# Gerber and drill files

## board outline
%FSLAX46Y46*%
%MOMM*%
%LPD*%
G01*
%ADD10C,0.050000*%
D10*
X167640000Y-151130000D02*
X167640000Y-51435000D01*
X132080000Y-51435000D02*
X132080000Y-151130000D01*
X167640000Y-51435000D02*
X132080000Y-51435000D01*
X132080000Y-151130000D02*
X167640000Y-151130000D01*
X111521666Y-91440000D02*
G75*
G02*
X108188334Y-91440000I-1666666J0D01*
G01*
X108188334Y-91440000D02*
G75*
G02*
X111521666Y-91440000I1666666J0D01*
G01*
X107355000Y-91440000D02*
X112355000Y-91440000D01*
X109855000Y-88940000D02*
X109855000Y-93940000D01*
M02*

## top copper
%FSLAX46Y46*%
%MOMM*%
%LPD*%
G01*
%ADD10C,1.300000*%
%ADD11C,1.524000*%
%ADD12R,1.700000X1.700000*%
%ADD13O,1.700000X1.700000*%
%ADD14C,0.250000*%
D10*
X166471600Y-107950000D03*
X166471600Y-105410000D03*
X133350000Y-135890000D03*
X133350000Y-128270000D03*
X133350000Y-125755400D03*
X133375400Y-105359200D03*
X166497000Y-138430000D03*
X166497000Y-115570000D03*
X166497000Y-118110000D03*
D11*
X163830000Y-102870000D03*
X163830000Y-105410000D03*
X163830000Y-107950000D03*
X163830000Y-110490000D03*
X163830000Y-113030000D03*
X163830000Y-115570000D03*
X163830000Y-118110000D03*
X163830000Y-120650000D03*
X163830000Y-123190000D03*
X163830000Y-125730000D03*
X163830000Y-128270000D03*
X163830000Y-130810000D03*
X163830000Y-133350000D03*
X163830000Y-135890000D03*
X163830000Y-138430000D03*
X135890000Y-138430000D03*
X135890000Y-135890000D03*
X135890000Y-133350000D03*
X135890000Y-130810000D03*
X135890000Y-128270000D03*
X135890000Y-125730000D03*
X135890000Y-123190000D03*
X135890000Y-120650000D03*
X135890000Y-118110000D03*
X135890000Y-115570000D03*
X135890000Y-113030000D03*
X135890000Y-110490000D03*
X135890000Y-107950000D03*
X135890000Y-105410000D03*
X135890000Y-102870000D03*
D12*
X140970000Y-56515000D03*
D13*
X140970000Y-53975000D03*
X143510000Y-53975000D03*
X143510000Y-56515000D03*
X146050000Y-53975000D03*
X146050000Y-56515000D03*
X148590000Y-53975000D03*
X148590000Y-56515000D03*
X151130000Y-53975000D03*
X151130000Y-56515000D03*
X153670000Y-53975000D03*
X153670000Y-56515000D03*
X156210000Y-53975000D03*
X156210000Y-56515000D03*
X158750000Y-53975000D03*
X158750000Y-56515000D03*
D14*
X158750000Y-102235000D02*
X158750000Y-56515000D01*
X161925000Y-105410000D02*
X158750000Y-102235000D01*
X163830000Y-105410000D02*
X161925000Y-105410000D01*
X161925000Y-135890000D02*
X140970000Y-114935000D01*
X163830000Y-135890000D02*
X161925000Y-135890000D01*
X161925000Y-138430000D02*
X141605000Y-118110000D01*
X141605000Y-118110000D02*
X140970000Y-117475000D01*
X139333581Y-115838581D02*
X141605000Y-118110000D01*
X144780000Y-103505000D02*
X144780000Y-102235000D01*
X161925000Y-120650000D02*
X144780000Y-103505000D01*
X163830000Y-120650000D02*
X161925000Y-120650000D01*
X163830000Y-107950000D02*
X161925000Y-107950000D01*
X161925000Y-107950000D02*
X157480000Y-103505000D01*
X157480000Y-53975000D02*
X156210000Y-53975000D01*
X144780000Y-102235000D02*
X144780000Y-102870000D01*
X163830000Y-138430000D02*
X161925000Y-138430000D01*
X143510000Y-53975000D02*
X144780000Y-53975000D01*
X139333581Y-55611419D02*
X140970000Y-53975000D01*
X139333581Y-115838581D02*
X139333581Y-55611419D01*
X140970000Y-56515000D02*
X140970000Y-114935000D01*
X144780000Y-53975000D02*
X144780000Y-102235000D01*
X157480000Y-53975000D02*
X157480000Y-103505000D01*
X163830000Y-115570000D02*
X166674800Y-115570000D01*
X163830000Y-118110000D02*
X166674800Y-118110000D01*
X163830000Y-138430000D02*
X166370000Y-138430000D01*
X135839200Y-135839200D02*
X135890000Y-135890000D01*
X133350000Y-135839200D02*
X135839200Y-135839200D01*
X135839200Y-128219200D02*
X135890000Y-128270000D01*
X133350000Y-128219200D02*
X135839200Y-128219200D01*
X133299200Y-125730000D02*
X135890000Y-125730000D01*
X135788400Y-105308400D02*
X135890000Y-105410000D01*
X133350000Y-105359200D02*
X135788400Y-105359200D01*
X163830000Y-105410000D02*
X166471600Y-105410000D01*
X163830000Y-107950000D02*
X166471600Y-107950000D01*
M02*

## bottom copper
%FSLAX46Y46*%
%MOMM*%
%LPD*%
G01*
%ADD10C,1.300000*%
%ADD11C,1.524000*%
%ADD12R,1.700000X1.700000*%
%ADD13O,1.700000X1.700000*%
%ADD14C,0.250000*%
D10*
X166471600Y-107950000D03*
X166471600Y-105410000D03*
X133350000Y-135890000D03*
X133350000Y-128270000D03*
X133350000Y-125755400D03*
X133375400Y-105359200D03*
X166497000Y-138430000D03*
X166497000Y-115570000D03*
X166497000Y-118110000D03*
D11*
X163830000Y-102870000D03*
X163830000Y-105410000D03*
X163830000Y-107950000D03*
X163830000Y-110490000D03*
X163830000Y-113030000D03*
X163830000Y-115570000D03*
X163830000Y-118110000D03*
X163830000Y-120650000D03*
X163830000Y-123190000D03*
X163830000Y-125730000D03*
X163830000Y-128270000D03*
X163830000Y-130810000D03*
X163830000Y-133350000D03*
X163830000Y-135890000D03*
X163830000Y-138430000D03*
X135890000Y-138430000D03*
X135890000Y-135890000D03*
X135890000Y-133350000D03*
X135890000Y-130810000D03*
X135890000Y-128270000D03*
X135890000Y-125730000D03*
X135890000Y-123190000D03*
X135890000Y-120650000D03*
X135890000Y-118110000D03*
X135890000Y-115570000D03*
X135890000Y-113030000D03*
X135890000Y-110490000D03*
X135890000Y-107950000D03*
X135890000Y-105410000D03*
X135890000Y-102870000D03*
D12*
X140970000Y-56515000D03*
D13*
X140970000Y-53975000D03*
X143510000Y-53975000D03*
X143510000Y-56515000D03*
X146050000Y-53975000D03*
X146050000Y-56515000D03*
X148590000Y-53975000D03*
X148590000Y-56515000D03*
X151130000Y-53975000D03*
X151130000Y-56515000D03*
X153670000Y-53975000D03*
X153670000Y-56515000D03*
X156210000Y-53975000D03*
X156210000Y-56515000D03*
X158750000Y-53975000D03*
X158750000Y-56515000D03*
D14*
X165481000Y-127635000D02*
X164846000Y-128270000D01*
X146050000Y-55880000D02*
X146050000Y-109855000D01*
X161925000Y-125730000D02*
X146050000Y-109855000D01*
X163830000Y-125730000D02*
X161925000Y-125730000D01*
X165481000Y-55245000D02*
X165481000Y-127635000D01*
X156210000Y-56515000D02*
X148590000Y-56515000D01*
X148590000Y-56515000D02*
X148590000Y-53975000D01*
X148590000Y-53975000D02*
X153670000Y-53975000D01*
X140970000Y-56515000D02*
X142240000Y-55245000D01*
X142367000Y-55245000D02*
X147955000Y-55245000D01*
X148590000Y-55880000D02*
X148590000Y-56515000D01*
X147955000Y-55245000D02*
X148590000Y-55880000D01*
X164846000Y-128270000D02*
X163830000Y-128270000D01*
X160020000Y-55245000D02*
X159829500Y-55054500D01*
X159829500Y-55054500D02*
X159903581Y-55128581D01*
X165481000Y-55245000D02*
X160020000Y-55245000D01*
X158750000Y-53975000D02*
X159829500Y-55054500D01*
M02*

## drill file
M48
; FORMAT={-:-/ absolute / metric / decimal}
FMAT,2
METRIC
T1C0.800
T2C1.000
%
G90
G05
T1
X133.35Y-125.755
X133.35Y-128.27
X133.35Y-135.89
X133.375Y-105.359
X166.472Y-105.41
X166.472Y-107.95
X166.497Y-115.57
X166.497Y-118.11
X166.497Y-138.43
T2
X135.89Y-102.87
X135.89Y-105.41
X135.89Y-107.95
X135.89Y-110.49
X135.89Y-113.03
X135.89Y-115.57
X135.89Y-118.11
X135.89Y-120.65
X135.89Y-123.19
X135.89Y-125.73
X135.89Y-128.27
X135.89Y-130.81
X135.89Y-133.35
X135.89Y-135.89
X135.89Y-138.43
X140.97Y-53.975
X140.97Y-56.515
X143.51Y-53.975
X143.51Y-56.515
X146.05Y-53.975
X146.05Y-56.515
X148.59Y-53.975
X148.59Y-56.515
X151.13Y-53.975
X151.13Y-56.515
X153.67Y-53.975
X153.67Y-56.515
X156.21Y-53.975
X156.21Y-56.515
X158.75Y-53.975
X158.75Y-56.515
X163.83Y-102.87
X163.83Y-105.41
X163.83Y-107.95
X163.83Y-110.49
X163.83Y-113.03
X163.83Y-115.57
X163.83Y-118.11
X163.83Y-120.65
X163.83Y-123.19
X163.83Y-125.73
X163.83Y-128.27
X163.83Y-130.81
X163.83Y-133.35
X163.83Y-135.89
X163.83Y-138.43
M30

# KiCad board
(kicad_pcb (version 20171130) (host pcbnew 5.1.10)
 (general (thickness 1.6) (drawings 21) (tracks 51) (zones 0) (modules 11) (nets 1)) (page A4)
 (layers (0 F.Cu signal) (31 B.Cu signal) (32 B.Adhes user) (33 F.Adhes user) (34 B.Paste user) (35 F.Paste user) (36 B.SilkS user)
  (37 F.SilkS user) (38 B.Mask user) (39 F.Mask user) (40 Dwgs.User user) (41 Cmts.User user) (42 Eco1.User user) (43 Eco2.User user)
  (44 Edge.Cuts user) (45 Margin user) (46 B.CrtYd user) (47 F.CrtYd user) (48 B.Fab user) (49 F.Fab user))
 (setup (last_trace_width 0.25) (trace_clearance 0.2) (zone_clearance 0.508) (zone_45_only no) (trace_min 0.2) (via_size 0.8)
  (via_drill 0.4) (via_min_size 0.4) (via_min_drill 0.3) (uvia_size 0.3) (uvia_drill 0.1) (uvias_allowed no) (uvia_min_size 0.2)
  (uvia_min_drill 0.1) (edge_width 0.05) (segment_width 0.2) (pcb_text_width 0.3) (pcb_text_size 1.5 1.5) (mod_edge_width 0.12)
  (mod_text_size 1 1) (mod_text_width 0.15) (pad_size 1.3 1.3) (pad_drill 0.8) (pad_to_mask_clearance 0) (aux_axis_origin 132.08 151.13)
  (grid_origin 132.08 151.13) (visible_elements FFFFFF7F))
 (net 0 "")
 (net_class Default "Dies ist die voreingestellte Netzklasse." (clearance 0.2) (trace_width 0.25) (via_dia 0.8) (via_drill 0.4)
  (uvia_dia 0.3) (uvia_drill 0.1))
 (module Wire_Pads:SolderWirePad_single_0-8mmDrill (layer F.Cu) (at 166.4716 107.95)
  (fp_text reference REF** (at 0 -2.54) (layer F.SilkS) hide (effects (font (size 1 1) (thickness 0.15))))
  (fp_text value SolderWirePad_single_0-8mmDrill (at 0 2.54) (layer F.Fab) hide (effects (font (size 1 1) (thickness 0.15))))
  (pad 1 thru_hole circle (at 0 0) (size 1.3 1.3) (drill 0.8) (layers *.Cu *.Mask)))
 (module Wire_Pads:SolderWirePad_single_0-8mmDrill (layer F.Cu) (at 166.4716 105.41)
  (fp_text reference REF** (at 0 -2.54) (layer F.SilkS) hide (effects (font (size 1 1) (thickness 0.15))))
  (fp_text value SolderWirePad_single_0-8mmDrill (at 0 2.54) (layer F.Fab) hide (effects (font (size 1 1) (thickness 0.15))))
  (pad 1 thru_hole circle (at 0 0) (size 1.3 1.3) (drill 0.8) (layers *.Cu *.Mask)))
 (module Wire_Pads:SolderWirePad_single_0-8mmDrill (layer F.Cu) (at 133.35 135.89)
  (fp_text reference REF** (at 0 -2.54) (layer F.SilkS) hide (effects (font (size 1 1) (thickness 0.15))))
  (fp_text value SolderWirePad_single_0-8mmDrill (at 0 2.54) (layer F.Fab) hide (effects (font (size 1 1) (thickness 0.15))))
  (pad 1 thru_hole circle (at 0 0) (size 1.3 1.3) (drill 0.8) (layers *.Cu *.Mask)))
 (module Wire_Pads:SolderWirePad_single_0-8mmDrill (layer F.Cu) (at 133.35 128.27)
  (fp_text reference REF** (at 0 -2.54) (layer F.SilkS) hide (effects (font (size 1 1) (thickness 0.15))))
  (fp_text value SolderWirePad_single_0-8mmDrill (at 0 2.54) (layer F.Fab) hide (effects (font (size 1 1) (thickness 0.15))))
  (pad 1 thru_hole circle (at 0 0) (size 1.3 1.3) (drill 0.8) (layers *.Cu *.Mask)))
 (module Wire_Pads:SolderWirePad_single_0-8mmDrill (layer F.Cu) (at 133.35 125.7554)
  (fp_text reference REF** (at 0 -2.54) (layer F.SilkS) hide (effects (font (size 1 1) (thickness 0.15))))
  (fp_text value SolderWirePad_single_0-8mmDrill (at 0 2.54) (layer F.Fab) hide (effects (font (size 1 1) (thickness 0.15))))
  (pad 1 thru_hole circle (at 0 0) (size 1.3 1.3) (drill 0.8) (layers *.Cu *.Mask)))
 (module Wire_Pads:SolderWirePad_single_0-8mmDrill (layer F.Cu) (at 133.3754 105.3592)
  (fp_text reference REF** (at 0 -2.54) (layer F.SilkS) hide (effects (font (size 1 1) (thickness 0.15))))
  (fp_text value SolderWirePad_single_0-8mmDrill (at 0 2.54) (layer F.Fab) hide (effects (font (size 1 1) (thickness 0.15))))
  (pad 1 thru_hole circle (at 0 0) (size 1.3 1.3) (drill 0.8) (layers *.Cu *.Mask)))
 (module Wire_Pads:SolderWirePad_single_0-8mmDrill (layer F.Cu) (at 166.497 138.43)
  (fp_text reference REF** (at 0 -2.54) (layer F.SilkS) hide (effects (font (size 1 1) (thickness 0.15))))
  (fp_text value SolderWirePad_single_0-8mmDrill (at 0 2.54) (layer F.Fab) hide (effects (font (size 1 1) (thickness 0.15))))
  (pad 1 thru_hole circle (at 0 0) (size 1.3 1.3) (drill 0.8) (layers *.Cu *.Mask)))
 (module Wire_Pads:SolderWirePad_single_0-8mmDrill (layer F.Cu) (at 166.497 115.57)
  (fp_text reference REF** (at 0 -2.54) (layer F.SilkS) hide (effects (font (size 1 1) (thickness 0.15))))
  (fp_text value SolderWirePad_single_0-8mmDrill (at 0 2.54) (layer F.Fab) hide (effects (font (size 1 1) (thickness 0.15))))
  (pad 1 thru_hole circle (at 0 0) (size 1.3 1.3) (drill 0.8) (layers *.Cu *.Mask)))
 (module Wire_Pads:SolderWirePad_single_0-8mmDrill (layer F.Cu) (at 166.497 118.11)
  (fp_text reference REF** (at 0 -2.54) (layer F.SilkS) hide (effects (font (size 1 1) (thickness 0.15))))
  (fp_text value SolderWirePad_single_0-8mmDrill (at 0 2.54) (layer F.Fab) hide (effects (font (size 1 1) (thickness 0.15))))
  (pad 1 thru_hole circle (at 0 0) (size 1.3 1.3) (drill 0.8) (layers *.Cu *.Mask)))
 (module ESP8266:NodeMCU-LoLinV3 (layer F.Cu) (at 149.86 123.19)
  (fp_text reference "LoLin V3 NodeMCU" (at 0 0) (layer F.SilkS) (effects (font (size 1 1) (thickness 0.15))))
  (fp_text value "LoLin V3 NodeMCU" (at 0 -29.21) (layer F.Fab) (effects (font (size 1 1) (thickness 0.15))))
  (pad 30 thru_hole circle (at 13.97 -20.32) (size 1.524 1.524) (drill 1) (layers *.Cu *.Mask F.SilkS))
  (pad 29 thru_hole circle (at 13.97 -17.78) (size 1.524 1.524) (drill 1) (layers *.Cu *.Mask F.SilkS))
  (pad 28 thru_hole circle (at 13.97 -15.24) (size 1.524 1.524) (drill 1) (layers *.Cu *.Mask F.SilkS))
  (pad 27 thru_hole circle (at 13.97 -12.7) (size 1.524 1.524) (drill 1) (layers *.Cu *.Mask F.SilkS))
  (pad 26 thru_hole circle (at 13.97 -10.16) (size 1.524 1.524) (drill 1) (layers *.Cu *.Mask F.SilkS))
  (pad 25 thru_hole circle (at 13.97 -7.62) (size 1.524 1.524) (drill 1) (layers *.Cu *.Mask F.SilkS))
  (pad 24 thru_hole circle (at 13.97 -5.08) (size 1.524 1.524) (drill 1) (layers *.Cu *.Mask F.SilkS))
  (pad 23 thru_hole circle (at 13.97 -2.54) (size 1.524 1.524) (drill 1) (layers *.Cu *.Mask F.SilkS))
  (pad 22 thru_hole circle (at 13.97 0) (size 1.524 1.524) (drill 1) (layers *.Cu *.Mask F.SilkS))
  (pad 21 thru_hole circle (at 13.97 2.54) (size 1.524 1.524) (drill 1) (layers *.Cu *.Mask F.SilkS))
  (pad 20 thru_hole circle (at 13.97 5.08) (size 1.524 1.524) (drill 1) (layers *.Cu *.Mask F.SilkS))
  (pad 19 thru_hole circle (at 13.97 7.62) (size 1.524 1.524) (drill 1) (layers *.Cu *.Mask F.SilkS))
  (pad 18 thru_hole circle (at 13.97 10.16) (size 1.524 1.524) (drill 1) (layers *.Cu *.Mask F.SilkS))
  (pad 17 thru_hole circle (at 13.97 12.7) (size 1.524 1.524) (drill 1) (layers *.Cu *.Mask F.SilkS))
  (pad 16 thru_hole circle (at 13.97 15.24) (size 1.524 1.524) (drill 1) (layers *.Cu *.Mask F.SilkS))
  (pad 15 thru_hole circle (at -13.97 15.24) (size 1.524 1.524) (drill 1) (layers *.Cu *.Mask F.SilkS))
  (pad 14 thru_hole circle (at -13.97 12.7) (size 1.524 1.524) (drill 1) (layers *.Cu *.Mask F.SilkS))
  (pad 13 thru_hole circle (at -13.97 10.16) (size 1.524 1.524) (drill 1) (layers *.Cu *.Mask F.SilkS))
  (pad 12 thru_hole circle (at -13.97 7.62) (size 1.524 1.524) (drill 1) (layers *.Cu *.Mask F.SilkS))
  (pad 11 thru_hole circle (at -13.97 5.08) (size 1.524 1.524) (drill 1) (layers *.Cu *.Mask F.SilkS))
  (pad 10 thru_hole circle (at -13.97 2.54) (size 1.524 1.524) (drill 1) (layers *.Cu *.Mask F.SilkS))
  (pad 9 thru_hole circle (at -13.97 0) (size 1.524 1.524) (drill 1) (layers *.Cu *.Mask F.SilkS))
  (pad 8 thru_hole circle (at -13.97 -2.54) (size 1.524 1.524) (drill 1) (layers *.Cu *.Mask F.SilkS))
  (pad 7 thru_hole circle (at -13.97 -5.08) (size 1.524 1.524) (drill 1) (layers *.Cu *.Mask F.SilkS))
  (pad 6 thru_hole circle (at -13.97 -7.62) (size 1.524 1.524) (drill 1) (layers *.Cu *.Mask F.SilkS))
  (pad 5 thru_hole circle (at -13.97 -10.16) (size 1.524 1.524) (drill 1) (layers *.Cu *.Mask F.SilkS))
  (pad 4 thru_hole circle (at -13.97 -12.7) (size 1.524 1.524) (drill 1) (layers *.Cu *.Mask F.SilkS))
  (pad 3 thru_hole circle (at -13.97 -15.24) (size 1.524 1.524) (drill 1) (layers *.Cu *.Mask F.SilkS))
  (pad 2 thru_hole circle (at -13.97 -17.78) (size 1.524 1.524) (drill 1) (layers *.Cu *.Mask F.SilkS))
  (pad 1 thru_hole circle (at -13.97 -20.32) (size 1.524 1.524) (drill 1) (layers *.Cu *.Mask F.SilkS)))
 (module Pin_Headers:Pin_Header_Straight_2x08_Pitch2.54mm (layer B.Cu) (at 140.97 53.975 270)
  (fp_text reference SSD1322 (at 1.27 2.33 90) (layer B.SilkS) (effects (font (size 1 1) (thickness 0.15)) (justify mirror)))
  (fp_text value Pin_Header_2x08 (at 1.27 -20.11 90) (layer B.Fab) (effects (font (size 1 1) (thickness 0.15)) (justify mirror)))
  (pad 1 thru_hole rect (at 2.54 0 270) (size 1.7 1.7) (drill 1) (layers *.Cu *.Mask))
  (pad 2 thru_hole oval (at 0 0 270) (size 1.7 1.7) (drill 1) (layers *.Cu *.Mask))
  (pad 4 thru_hole oval (at 0 -2.54 270) (size 1.7 1.7) (drill 1) (layers *.Cu *.Mask))
  (pad 3 thru_hole oval (at 2.54 -2.54 270) (size 1.7 1.7) (drill 1) (layers *.Cu *.Mask))
  (pad 6 thru_hole oval (at 0 -5.08 270) (size 1.7 1.7) (drill 1) (layers *.Cu *.Mask))
  (pad 5 thru_hole oval (at 2.54 -5.08 270) (size 1.7 1.7) (drill 1) (layers *.Cu *.Mask))
  (pad 8 thru_hole oval (at 0 -7.62 270) (size 1.7 1.7) (drill 1) (layers *.Cu *.Mask))
  (pad 7 thru_hole oval (at 2.54 -7.62 270) (size 1.7 1.7) (drill 1) (layers *.Cu *.Mask))
  (pad 10 thru_hole oval (at 0 -10.16 270) (size 1.7 1.7) (drill 1) (layers *.Cu *.Mask))
  (pad 9 thru_hole oval (at 2.54 -10.16 270) (size 1.7 1.7) (drill 1) (layers *.Cu *.Mask))
  (pad 12 thru_hole oval (at 0 -12.7 270) (size 1.7 1.7) (drill 1) (layers *.Cu *.Mask))
  (pad 11 thru_hole oval (at 2.54 -12.7 270) (size 1.7 1.7) (drill 1) (layers *.Cu *.Mask))
  (pad 14 thru_hole oval (at 0 -15.24 270) (size 1.7 1.7) (drill 1) (layers *.Cu *.Mask))
  (pad 13 thru_hole oval (at 2.54 -15.24 270) (size 1.7 1.7) (drill 1) (layers *.Cu *.Mask))
  (pad 16 thru_hole oval (at 0 -17.78 270) (size 1.7 1.7) (drill 1) (layers *.Cu *.Mask))
  (pad 15 thru_hole oval (at 2.54 -17.78 270) (size 1.7 1.7) (drill 1) (layers *.Cu *.Mask)))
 (gr_line (start 167.64 151.13) (end 167.64 51.435) (layer Edge.Cuts) (width 0.05))
 (gr_line (start 132.08 51.435) (end 132.08 151.13) (layer Edge.Cuts) (width 0.05))
 (gr_line (start 167.64 51.435) (end 132.08 51.435) (layer Edge.Cuts) (width 0.05))
 (gr_line (start 132.08 151.13) (end 167.64 151.13) (layer Edge.Cuts) (width 0.05))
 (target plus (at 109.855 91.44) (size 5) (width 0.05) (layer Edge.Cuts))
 (segment (start 165.481 127.635) (end 164.846 128.27) (width 0.25) (layer B.Cu) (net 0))
 (segment (start 158.75 102.235) (end 158.75 56.515) (width 0.25) (layer F.Cu) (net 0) (status 20))
 (segment (start 161.925 105.41) (end 158.75 102.235) (width 0.25) (layer F.Cu) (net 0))
 (segment (start 163.83 105.41) (end 161.925 105.41) (width 0.25) (layer F.Cu) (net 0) (status 10))
 (segment (start 161.925 135.89) (end 140.97 114.935) (width 0.25) (layer F.Cu) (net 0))
 (segment (start 163.83 135.89) (end 161.925 135.89) (width 0.25) (layer F.Cu) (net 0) (status 10))
 (segment (start 161.925 138.43) (end 141.605 118.11) (width 0.25) (layer F.Cu) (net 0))
 (segment (start 141.605 118.11) (end 140.97 117.475) (width 0.25) (layer F.Cu) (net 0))
 (segment (start 139.333581 115.838581) (end 141.605 118.11) (width 0.25) (layer F.Cu) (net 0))
 (segment (start 144.78 103.505) (end 144.78 102.235) (width 0.25) (layer F.Cu) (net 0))
 (segment (start 161.925 120.65) (end 144.78 103.505) (width 0.25) (layer F.Cu) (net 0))
 (segment (start 163.83 120.65) (end 161.925 120.65) (width 0.25) (layer F.Cu) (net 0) (status 10))
 (segment (start 146.05 55.88) (end 146.05 109.855) (width 0.25) (layer B.Cu) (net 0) (status 10))
 (segment (start 161.925 125.73) (end 146.05 109.855) (width 0.25) (layer B.Cu) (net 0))
 (segment (start 163.83 125.73) (end 161.925 125.73) (width 0.25) (layer B.Cu) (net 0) (status 10))
 (segment (start 163.83 107.95) (end 161.925 107.95) (width 0.25) (layer F.Cu) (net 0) (status 10))
 (segment (start 161.925 107.95) (end 157.48 103.505) (width 0.25) (layer F.Cu) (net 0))
 (segment (start 157.48 53.975) (end 156.21 53.975) (width 0.25) (layer F.Cu) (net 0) (status 20))
 (segment (start 144.78 102.235) (end 144.78 102.87) (width 0.25) (layer F.Cu) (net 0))
 (segment (start 163.83 138.43) (end 161.925 138.43) (width 0.25) (layer F.Cu) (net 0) (status 10))
 (segment (start 143.51 53.975) (end 144.78 53.975) (width 0.25) (layer F.Cu) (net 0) (status 10))
 (segment (start 139.333581 55.611419) (end 140.97 53.975) (width 0.25) (layer F.Cu) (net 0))
 (segment (start 139.333581 115.838581) (end 139.333581 55.611419) (width 0.25) (layer F.Cu) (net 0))
 (segment (start 140.97 56.515) (end 140.97 114.935) (width 0.25) (layer F.Cu) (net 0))
 (segment (start 144.78 53.975) (end 144.78 102.235) (width 0.25) (layer F.Cu) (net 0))
 (segment (start 157.48 53.975) (end 157.48 103.505) (width 0.25) (layer F.Cu) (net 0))
 (segment (start 165.481 55.245) (end 165.481 127.635) (width 0.25) (layer B.Cu) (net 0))
 (segment (start 156.21 56.515) (end 148.59 56.515) (width 0.25) (layer B.Cu) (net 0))
 (segment (start 148.59 56.515) (end 148.59 53.975) (width 0.25) (layer B.Cu) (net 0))
 (segment (start 148.59 53.975) (end 153.67 53.975) (width 0.25) (layer B.Cu) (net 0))
 (segment (start 140.97 56.515) (end 142.24 55.245) (width 0.25) (layer B.Cu) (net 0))
 (segment (start 142.367 55.245) (end 147.955 55.245) (width 0.25) (layer B.Cu) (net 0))
 (segment (start 148.59 55.88) (end 148.59 56.515) (width 0.25) (layer B.Cu) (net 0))
 (segment (start 147.955 55.245) (end 148.59 55.88) (width 0.25) (layer B.Cu) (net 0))
 (segment (start 163.83 115.57) (end 166.6748 115.57) (width 0.25) (layer F.Cu) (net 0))
 (segment (start 163.83 118.11) (end 166.6748 118.11) (width 0.25) (layer F.Cu) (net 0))
 (segment (start 163.83 138.43) (end 166.37 138.43) (width 0.25) (layer F.Cu) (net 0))
 (segment (start 135.8392 135.8392) (end 135.89 135.89) (width 0.25) (layer F.Cu) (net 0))
 (segment (start 133.35 135.8392) (end 135.8392 135.8392) (width 0.25) (layer F.Cu) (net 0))
 (segment (start 135.8392 128.2192) (end 135.89 128.27) (width 0.25) (layer F.Cu) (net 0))
 (segment (start 133.35 128.2192) (end 135.8392 128.2192) (width 0.25) (layer F.Cu) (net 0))
 (segment (start 133.2992 125.73) (end 135.89 125.73) (width 0.25) (layer F.Cu) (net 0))
 (segment (start 135.7884 105.3084) (end 135.89 105.41) (width 0.25) (layer F.Cu) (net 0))
 (segment (start 133.35 105.3592) (end 135.7884 105.3592) (width 0.25) (layer F.Cu) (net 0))
 (segment (start 164.846 128.27) (end 163.83 128.27) (width 0.25) (layer B.Cu) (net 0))
 (segment (start 160.02 55.245) (end 159.8295 55.0545) (width 0.25) (layer B.Cu) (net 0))
 (segment (start 159.8295 55.0545) (end 159.903581 55.128581) (width 0.25) (layer B.Cu) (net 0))
 (segment (start 165.481 55.245) (end 160.02 55.245) (width 0.25) (layer B.Cu) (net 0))
 (segment (start 158.75 53.975) (end 159.8295 55.0545) (width 0.25) (layer B.Cu) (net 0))
 (segment (start 163.83 105.41) (end 166.4716 105.41) (width 0.25) (layer F.Cu) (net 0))
 (segment (start 163.83 107.95) (end 166.4716 107.95) (width 0.25) (layer F.Cu) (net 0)))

